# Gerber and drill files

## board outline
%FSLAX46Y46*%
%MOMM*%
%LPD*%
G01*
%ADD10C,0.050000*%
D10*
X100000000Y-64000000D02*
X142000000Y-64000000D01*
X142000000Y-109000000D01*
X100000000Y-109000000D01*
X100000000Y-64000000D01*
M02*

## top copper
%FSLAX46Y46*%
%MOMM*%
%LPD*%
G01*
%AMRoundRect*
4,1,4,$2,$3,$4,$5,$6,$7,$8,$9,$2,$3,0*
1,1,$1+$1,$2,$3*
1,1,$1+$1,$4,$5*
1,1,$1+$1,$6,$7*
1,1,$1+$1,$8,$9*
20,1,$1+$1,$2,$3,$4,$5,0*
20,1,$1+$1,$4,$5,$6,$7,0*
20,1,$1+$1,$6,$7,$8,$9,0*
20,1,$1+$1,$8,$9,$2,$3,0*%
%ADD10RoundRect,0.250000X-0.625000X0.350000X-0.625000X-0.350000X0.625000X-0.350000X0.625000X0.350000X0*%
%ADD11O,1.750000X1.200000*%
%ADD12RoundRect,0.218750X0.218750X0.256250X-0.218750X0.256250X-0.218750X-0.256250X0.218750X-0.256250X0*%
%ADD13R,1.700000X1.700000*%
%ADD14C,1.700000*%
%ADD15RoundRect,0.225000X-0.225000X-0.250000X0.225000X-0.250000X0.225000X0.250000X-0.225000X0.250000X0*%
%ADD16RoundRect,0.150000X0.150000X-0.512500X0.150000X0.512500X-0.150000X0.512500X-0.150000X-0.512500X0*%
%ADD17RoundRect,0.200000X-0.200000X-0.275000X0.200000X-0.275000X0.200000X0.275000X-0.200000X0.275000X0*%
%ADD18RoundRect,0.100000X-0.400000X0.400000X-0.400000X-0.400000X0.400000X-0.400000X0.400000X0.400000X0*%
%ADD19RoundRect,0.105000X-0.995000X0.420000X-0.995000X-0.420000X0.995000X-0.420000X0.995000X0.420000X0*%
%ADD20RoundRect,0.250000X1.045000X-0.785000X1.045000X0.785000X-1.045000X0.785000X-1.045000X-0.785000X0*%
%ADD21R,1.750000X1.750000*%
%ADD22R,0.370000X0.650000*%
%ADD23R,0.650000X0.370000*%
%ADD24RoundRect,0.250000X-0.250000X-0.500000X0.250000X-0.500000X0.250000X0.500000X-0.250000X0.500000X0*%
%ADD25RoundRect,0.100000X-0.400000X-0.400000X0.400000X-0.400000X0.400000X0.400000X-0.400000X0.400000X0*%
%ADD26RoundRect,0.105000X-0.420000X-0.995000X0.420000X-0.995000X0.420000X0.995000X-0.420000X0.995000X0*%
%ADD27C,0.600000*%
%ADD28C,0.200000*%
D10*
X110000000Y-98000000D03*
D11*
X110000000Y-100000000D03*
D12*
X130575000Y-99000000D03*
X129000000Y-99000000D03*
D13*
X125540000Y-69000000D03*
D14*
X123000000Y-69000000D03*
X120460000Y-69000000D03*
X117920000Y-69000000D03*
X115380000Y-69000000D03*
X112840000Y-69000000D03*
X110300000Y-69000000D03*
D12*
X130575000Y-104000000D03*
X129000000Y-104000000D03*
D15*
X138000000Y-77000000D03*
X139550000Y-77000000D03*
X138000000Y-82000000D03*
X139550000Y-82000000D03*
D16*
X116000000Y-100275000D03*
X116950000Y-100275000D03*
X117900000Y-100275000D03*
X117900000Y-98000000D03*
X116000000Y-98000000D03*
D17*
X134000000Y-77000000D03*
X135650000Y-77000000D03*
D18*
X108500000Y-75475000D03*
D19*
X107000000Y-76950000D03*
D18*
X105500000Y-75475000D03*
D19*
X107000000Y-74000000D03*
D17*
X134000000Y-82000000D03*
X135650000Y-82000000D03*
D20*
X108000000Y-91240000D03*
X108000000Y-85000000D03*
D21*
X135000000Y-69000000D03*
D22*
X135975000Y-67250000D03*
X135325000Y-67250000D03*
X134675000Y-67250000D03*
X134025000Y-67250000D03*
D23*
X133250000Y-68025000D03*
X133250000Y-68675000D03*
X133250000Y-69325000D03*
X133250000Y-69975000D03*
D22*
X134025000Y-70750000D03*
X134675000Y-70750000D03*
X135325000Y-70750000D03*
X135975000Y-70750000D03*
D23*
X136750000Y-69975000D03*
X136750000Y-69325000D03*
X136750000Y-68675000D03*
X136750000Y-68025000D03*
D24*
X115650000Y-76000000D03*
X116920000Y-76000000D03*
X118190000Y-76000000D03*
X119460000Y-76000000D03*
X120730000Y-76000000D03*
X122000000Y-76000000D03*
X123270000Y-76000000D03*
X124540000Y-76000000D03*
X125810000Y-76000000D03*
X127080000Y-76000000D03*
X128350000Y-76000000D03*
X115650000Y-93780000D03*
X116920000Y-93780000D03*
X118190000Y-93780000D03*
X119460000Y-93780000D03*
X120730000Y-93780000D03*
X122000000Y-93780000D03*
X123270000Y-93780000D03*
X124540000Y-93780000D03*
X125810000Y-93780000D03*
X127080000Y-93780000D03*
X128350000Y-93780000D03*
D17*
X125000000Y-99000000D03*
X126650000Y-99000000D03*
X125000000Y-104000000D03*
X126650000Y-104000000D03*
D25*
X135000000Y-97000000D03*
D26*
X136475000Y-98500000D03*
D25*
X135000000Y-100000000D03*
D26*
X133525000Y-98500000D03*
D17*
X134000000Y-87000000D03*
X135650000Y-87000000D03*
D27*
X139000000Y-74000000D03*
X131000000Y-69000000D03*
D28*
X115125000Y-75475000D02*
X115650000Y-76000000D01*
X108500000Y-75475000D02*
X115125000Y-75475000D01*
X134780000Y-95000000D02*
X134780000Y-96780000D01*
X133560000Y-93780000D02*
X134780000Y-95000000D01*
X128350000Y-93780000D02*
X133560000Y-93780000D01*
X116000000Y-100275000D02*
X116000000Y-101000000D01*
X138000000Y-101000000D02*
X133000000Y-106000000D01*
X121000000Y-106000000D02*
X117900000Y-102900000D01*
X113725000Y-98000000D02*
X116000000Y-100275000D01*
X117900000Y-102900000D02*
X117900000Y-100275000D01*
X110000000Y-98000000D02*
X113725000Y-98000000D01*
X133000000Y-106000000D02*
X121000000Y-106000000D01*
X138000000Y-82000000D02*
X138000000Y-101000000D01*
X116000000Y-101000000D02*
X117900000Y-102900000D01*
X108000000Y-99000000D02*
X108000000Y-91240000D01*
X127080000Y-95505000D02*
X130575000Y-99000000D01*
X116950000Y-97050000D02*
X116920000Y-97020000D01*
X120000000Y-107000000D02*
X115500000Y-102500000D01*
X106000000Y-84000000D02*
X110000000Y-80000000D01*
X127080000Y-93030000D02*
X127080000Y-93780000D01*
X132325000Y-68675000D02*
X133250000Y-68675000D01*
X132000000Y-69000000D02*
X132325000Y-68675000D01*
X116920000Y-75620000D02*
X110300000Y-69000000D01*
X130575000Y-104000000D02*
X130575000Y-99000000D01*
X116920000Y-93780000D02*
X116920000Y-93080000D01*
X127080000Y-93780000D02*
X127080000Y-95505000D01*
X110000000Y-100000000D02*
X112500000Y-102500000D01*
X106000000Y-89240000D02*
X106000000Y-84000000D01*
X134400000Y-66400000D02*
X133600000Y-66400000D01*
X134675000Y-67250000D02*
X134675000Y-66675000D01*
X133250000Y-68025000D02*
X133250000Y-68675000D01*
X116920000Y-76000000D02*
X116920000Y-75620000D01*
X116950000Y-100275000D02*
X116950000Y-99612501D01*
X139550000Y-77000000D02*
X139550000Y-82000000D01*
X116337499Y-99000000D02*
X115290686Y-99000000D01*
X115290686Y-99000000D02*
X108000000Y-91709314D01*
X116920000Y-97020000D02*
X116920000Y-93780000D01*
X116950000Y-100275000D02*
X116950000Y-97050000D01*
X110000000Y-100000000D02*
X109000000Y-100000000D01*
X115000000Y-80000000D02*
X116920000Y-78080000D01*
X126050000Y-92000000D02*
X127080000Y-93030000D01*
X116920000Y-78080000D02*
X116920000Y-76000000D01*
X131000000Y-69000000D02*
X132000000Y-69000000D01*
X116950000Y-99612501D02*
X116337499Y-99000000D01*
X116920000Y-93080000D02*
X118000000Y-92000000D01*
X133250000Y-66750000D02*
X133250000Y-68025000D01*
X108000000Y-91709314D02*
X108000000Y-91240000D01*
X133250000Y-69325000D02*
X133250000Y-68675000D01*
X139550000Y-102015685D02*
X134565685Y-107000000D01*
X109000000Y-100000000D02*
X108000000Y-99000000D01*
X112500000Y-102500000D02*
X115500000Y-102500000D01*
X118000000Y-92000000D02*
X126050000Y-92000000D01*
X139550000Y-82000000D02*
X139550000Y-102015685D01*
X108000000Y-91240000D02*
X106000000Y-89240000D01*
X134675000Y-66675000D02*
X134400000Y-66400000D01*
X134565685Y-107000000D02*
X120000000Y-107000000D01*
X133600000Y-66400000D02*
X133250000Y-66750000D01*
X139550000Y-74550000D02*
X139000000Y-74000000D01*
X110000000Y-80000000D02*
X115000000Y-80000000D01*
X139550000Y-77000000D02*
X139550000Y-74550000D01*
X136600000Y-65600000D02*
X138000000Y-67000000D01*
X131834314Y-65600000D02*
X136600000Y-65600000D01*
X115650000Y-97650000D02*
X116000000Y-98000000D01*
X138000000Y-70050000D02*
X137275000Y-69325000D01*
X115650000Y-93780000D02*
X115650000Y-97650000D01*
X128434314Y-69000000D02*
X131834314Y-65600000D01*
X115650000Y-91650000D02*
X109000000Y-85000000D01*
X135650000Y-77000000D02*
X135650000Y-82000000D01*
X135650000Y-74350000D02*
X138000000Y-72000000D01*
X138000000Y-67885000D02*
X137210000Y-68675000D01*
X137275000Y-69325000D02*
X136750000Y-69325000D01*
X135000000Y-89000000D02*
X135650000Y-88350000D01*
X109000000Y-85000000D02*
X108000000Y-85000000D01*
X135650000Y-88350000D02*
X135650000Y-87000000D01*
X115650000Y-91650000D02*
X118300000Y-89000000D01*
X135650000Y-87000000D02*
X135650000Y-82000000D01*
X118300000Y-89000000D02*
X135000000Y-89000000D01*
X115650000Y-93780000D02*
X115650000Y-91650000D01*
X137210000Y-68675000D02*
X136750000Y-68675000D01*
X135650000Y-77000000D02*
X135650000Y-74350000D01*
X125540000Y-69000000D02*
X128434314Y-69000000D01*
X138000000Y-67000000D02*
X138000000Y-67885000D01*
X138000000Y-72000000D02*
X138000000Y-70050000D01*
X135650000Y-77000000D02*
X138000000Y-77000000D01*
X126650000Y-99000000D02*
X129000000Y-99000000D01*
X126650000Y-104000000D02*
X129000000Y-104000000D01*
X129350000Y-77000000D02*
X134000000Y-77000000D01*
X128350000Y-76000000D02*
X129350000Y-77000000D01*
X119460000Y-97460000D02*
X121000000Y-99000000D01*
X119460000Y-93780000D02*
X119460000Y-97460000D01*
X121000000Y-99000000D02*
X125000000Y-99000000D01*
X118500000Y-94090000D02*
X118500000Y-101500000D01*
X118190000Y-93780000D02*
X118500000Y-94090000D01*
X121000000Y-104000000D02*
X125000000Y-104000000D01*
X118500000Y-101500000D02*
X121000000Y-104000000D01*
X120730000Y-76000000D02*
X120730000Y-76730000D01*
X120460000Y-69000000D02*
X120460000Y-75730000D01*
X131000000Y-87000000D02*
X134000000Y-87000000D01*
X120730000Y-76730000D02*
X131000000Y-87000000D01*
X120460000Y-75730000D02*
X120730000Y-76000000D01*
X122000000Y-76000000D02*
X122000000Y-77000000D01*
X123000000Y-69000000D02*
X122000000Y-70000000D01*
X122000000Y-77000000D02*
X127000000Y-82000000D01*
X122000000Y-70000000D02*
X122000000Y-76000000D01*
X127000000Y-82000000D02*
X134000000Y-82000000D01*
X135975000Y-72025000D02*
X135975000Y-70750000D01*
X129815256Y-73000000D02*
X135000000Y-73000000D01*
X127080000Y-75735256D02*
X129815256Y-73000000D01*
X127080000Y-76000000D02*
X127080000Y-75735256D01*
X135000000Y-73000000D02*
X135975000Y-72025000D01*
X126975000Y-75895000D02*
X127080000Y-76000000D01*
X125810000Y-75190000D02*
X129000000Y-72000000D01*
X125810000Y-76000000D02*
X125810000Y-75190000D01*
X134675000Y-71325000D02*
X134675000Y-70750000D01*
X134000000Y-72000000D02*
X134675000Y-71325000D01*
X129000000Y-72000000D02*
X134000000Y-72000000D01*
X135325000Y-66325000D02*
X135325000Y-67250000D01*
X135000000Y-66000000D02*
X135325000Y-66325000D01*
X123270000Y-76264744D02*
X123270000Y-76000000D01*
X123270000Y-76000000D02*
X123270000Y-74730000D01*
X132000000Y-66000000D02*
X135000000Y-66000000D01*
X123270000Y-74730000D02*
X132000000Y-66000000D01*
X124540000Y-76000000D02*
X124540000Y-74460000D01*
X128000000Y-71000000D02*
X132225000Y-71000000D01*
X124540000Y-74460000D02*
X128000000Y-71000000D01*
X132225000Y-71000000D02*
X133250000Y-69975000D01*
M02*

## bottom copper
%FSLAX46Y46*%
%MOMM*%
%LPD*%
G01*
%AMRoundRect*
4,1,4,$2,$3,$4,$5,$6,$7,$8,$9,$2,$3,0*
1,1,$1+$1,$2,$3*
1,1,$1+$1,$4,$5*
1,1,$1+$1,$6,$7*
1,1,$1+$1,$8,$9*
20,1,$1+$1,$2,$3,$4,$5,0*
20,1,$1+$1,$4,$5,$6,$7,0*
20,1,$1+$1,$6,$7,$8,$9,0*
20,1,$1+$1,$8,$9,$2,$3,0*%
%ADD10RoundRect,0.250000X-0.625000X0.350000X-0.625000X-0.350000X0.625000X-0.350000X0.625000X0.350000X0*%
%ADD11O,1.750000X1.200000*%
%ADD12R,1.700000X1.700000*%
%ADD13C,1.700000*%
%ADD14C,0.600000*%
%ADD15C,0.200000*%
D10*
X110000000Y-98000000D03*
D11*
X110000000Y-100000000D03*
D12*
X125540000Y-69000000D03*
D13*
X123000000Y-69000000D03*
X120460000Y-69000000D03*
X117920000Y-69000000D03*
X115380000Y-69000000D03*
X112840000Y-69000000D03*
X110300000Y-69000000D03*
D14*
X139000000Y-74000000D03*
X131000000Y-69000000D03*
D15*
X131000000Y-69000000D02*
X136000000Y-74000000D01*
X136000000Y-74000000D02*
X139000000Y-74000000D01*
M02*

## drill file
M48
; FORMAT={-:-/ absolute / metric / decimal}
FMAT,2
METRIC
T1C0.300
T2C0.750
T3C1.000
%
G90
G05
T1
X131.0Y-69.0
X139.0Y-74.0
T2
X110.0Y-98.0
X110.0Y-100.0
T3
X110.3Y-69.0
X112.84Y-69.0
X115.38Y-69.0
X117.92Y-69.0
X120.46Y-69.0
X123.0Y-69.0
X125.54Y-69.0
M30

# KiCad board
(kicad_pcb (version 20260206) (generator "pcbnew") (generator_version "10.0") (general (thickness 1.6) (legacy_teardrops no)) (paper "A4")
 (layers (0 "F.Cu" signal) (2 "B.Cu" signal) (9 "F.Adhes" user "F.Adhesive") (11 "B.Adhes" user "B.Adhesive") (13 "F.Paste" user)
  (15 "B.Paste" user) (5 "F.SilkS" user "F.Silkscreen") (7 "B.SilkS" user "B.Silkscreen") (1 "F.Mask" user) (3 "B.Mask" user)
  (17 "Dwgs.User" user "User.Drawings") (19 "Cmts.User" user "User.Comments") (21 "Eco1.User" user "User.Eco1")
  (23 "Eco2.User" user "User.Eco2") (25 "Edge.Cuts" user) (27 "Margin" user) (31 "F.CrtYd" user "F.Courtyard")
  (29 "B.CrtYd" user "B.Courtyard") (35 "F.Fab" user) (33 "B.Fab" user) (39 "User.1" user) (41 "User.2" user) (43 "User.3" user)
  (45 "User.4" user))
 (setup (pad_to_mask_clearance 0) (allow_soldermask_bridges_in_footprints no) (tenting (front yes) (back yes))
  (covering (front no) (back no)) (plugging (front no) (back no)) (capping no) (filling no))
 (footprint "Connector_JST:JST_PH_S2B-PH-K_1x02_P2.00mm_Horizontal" (layer "F.Cu") (at 110 98 -90)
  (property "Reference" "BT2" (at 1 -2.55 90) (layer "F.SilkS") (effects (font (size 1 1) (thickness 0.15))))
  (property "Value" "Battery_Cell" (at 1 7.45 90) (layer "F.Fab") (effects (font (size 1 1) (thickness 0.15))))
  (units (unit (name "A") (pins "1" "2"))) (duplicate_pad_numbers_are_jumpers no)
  (pad "1" thru_hole roundrect (at 0 0 270) (size 1.2 1.75) (drill 0.75) (layers "*.Cu" "*.Mask") (remove_unused_layers no)
   (roundrect_rratio 0.208333) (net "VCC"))
  (pad "2" thru_hole oval (at 2 0 270) (size 1.2 1.75) (drill 0.75) (layers "*.Cu" "*.Mask") (remove_unused_layers no) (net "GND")))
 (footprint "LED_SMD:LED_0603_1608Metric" (layer "F.Cu") (at 129.7875 99 180)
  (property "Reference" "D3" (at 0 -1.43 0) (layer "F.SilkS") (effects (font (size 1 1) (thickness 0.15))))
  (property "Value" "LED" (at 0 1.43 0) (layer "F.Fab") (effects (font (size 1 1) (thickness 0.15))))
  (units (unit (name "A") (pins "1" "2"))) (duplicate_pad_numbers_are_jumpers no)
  (pad "1" smd roundrect (at -0.7875 0 180) (size 0.875 0.95) (layers "F.Cu" "F.Mask" "F.Paste") (roundrect_rratio 0.25) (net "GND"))
  (pad "2" smd roundrect (at 0.7875 0 180) (size 0.875 0.95) (layers "F.Cu" "F.Mask" "F.Paste") (roundrect_rratio 0.25) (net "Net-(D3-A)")))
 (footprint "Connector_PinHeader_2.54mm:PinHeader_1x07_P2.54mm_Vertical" (layer "F.Cu") (at 125.54 69 -90)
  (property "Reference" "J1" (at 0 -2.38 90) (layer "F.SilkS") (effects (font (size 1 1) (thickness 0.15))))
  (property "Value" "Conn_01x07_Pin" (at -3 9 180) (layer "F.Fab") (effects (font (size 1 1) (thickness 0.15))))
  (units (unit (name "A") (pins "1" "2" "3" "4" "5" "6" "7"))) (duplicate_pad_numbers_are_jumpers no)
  (pad "1" thru_hole rect (at 0 0 270) (size 1.7 1.7) (drill 1) (layers "*.Cu" "*.Mask") (remove_unused_layers no) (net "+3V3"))
  (pad "2" thru_hole circle (at 0 2.54 270) (size 1.7 1.7) (drill 1) (layers "*.Cu" "*.Mask") (remove_unused_layers no)
   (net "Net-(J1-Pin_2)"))
  (pad "3" thru_hole circle (at 0 5.08 270) (size 1.7 1.7) (drill 1) (layers "*.Cu" "*.Mask") (remove_unused_layers no)
   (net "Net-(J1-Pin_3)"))
  (pad "4" thru_hole circle (at 0 7.62 270) (size 1.7 1.7) (drill 1) (layers "*.Cu" "*.Mask") (remove_unused_layers no)
   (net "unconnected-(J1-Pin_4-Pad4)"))
  (pad "5" thru_hole circle (at 0 10.16 270) (size 1.7 1.7) (drill 1) (layers "*.Cu" "*.Mask") (remove_unused_layers no)
   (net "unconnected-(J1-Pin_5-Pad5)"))
  (pad "6" thru_hole circle (at 0 12.7 270) (size 1.7 1.7) (drill 1) (layers "*.Cu" "*.Mask") (remove_unused_layers no)
   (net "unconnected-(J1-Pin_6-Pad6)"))
  (pad "7" thru_hole circle (at 0 15.24 270) (size 1.7 1.7) (drill 1) (layers "*.Cu" "*.Mask") (remove_unused_layers no) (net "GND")))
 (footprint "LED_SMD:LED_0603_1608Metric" (layer "F.Cu") (at 129.7875 104 180)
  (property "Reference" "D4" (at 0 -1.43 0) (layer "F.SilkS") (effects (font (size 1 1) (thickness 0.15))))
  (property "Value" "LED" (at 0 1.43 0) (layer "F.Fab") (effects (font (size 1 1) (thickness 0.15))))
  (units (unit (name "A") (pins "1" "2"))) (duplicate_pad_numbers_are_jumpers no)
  (pad "1" smd roundrect (at -0.7875 0 180) (size 0.875 0.95) (layers "F.Cu" "F.Mask" "F.Paste") (roundrect_rratio 0.25) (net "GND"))
  (pad "2" smd roundrect (at 0.7875 0 180) (size 0.875 0.95) (layers "F.Cu" "F.Mask" "F.Paste") (roundrect_rratio 0.25) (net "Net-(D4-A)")))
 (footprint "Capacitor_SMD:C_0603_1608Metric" (layer "F.Cu") (at 138.775 77)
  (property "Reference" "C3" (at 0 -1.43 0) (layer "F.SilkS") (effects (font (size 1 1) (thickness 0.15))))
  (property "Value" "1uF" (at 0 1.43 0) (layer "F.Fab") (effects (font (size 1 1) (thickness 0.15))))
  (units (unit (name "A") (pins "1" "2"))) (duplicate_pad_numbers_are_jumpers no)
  (pad "1" smd roundrect (at -0.775 0) (size 0.9 0.95) (layers "F.Cu" "F.Mask" "F.Paste") (roundrect_rratio 0.25) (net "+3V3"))
  (pad "2" smd roundrect (at 0.775 0) (size 0.9 0.95) (layers "F.Cu" "F.Mask" "F.Paste") (roundrect_rratio 0.25) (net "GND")))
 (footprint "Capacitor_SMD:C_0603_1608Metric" (layer "F.Cu") (at 138.775 82)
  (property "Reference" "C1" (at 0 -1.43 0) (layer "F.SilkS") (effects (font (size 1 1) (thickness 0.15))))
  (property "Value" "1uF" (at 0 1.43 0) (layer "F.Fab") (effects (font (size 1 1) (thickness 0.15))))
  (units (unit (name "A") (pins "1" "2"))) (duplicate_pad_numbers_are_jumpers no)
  (pad "1" smd roundrect (at -0.775 0) (size 0.9 0.95) (layers "F.Cu" "F.Mask" "F.Paste") (roundrect_rratio 0.25) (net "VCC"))
  (pad "2" smd roundrect (at 0.775 0) (size 0.9 0.95) (layers "F.Cu" "F.Mask" "F.Paste") (roundrect_rratio 0.25) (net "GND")))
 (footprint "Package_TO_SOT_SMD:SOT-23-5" (layer "F.Cu") (at 116.95 99.1375 90)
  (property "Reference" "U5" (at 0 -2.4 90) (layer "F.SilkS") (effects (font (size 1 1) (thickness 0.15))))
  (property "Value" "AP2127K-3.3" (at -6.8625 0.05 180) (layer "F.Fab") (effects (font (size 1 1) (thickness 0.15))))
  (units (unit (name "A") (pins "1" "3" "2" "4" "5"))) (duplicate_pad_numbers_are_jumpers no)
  (pad "1" smd roundrect (at -1.1375 -0.95 90) (size 1.325 0.6) (layers "F.Cu" "F.Mask" "F.Paste") (roundrect_rratio 0.25) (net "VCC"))
  (pad "2" smd roundrect (at -1.1375 0 90) (size 1.325 0.6) (layers "F.Cu" "F.Mask" "F.Paste") (roundrect_rratio 0.25) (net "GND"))
  (pad "3" smd roundrect (at -1.1375 0.95 90) (size 1.325 0.6) (layers "F.Cu" "F.Mask" "F.Paste") (roundrect_rratio 0.25) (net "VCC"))
  (pad "4" smd roundrect (at 1.1375 0.95 90) (size 1.325 0.6) (layers "F.Cu" "F.Mask" "F.Paste") (roundrect_rratio 0.25)
   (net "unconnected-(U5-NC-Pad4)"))
  (pad "5" smd roundrect (at 1.1375 -0.95 90) (size 1.325 0.6) (layers "F.Cu" "F.Mask" "F.Paste") (roundrect_rratio 0.25) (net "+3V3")))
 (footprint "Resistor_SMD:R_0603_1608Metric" (layer "F.Cu") (at 134.825 77)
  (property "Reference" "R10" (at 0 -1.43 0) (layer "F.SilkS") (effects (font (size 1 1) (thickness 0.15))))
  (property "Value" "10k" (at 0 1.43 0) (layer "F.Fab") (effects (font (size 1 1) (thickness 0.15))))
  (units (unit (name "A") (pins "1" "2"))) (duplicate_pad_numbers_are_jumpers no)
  (pad "1" smd roundrect (at -0.825 0) (size 0.8 0.95) (layers "F.Cu" "F.Mask" "F.Paste") (roundrect_rratio 0.25) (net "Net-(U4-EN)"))
  (pad "2" smd roundrect (at 0.825 0) (size 0.8 0.95) (layers "F.Cu" "F.Mask" "F.Paste") (roundrect_rratio 0.25) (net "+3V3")))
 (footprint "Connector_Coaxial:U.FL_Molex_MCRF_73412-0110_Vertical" (layer "F.Cu") (at 107 75.475 90)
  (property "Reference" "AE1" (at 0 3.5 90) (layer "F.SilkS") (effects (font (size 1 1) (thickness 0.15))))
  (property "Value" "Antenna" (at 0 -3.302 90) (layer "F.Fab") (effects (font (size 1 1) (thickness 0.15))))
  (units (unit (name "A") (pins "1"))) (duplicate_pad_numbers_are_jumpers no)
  (pad "1" smd roundrect (at 0 1.5 270) (size 1 1) (layers "F.Cu" "F.Mask" "F.Paste") (roundrect_rratio 0.1) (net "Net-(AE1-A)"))
  (pad "2" smd roundrect (at -1.475 0 270) (size 1.05 2.2) (layers "F.Cu" "F.Mask" "F.Paste") (roundrect_rratio 0.1))
  (pad "2" smd roundrect (at 0 -1.5 270) (size 1 1) (layers "F.Cu" "F.Mask" "F.Paste") (roundrect_rratio 0.1))
  (pad "2" smd roundrect (at 1.475 0 270) (size 1.05 2.2) (layers "F.Cu" "F.Mask" "F.Paste") (roundrect_rratio 0.1)))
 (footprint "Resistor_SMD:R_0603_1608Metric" (layer "F.Cu") (at 134.825 82)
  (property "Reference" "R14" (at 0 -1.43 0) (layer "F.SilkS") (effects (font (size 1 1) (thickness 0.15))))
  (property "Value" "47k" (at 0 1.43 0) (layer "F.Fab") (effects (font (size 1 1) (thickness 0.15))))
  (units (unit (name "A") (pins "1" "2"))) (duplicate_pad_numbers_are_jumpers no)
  (pad "1" smd roundrect (at -0.825 0) (size 0.8 0.95) (layers "F.Cu" "F.Mask" "F.Paste") (roundrect_rratio 0.25) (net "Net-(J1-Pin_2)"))
  (pad "2" smd roundrect (at 0.825 0) (size 0.8 0.95) (layers "F.Cu" "F.Mask" "F.Paste") (roundrect_rratio 0.25) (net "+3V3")))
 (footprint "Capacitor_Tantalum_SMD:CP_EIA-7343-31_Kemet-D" (layer "F.Cu") (at 108 88.12 90)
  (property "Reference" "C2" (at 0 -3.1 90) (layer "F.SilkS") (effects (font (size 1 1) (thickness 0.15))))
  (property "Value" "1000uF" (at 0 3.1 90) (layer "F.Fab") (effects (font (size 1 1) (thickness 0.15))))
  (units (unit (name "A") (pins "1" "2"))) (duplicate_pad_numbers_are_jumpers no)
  (pad "1" smd roundrect (at -3.12 0 90) (size 2.07 2.59) (layers "F.Cu" "F.Mask" "F.Paste") (roundrect_rratio 0.120773) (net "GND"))
  (pad "2" smd roundrect (at 3.12 0 90) (size 2.07 2.59) (layers "F.Cu" "F.Mask" "F.Paste") (roundrect_rratio 0.120773) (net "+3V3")))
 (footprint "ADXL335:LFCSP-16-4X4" (layer "F.Cu") (at 135 69 -90)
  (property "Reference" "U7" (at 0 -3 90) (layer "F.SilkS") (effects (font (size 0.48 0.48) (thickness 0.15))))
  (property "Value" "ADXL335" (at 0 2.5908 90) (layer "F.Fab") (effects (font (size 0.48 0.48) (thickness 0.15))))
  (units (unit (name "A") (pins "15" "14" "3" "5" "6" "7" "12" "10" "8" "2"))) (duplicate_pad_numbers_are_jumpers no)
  (pad "0" smd rect (at 0 0 270) (size 1.75 1.75) (layers "F.Cu" "F.Mask") (solder_mask_margin 0.102))
  (pad "1" smd rect (at -1.75 -0.975 270) (size 0.65 0.37) (layers "F.Cu" "F.Mask" "F.Paste") (solder_mask_margin 0.102))
  (pad "2" smd rect (at -1.75 -0.325 270) (size 0.65 0.37) (layers "F.Cu" "F.Mask" "F.Paste") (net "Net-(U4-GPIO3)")
   (solder_mask_margin 0.102))
  (pad "3" smd rect (at -1.75 0.325 270) (size 0.65 0.37) (layers "F.Cu" "F.Mask" "F.Paste") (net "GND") (solder_mask_margin 0.102))
  (pad "4" smd rect (at -1.75 0.975 270) (size 0.65 0.37) (layers "F.Cu" "F.Mask" "F.Paste") (solder_mask_margin 0.102))
  (pad "5" smd rect (at -0.975 1.75 270) (size 0.37 0.65) (layers "F.Cu" "F.Mask" "F.Paste") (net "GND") (solder_mask_margin 0.102))
  (pad "6" smd rect (at -0.325 1.75 270) (size 0.37 0.65) (layers "F.Cu" "F.Mask" "F.Paste") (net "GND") (solder_mask_margin 0.102))
  (pad "7" smd rect (at 0.325 1.75 270) (size 0.37 0.65) (layers "F.Cu" "F.Mask" "F.Paste") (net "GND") (solder_mask_margin 0.102))
  (pad "8" smd rect (at 0.975 1.75 270) (size 0.37 0.65) (layers "F.Cu" "F.Mask" "F.Paste") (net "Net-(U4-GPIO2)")
   (solder_mask_margin 0.102))
  (pad "9" smd rect (at 1.75 0.975 270) (size 0.65 0.37) (layers "F.Cu" "F.Mask" "F.Paste") (solder_mask_margin 0.102))
  (pad "10" smd rect (at 1.75 0.325 270) (size 0.65 0.37) (layers "F.Cu" "F.Mask" "F.Paste") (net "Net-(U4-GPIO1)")
   (solder_mask_margin 0.102))
  (pad "11" smd rect (at 1.75 -0.325 270) (size 0.65 0.37) (layers "F.Cu" "F.Mask" "F.Paste") (solder_mask_margin 0.102))
  (pad "12" smd rect (at 1.75 -0.975 270) (size 0.65 0.37) (layers "F.Cu" "F.Mask" "F.Paste") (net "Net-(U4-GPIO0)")
   (solder_mask_margin 0.102))
  (pad "13" smd rect (at 0.975 -1.75 270) (size 0.37 0.65) (layers "F.Cu" "F.Mask" "F.Paste") (solder_mask_margin 0.102))
  (pad "14" smd rect (at 0.325 -1.75 270) (size 0.37 0.65) (layers "F.Cu" "F.Mask" "F.Paste") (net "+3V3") (solder_mask_margin 0.102))
  (pad "15" smd rect (at -0.325 -1.75 270) (size 0.37 0.65) (layers "F.Cu" "F.Mask" "F.Paste") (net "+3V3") (solder_mask_margin 0.102))
  (pad "16" smd rect (at -0.975 -1.75 270) (size 0.37 0.65) (layers "F.Cu" "F.Mask" "F.Paste") (solder_mask_margin 0.102)))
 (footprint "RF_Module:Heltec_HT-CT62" (layer "F.Cu") (at 122 84.89)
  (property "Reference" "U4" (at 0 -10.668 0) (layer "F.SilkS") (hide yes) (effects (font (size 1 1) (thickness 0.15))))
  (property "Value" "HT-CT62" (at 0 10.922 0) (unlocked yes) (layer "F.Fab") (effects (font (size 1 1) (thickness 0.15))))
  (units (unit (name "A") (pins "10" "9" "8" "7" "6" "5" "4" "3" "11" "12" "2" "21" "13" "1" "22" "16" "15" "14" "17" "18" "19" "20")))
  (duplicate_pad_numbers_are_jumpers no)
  (pad "1" smd roundrect (at -6.35 -8.89) (size 1 1.5) (layers "F.Cu" "F.Mask" "F.Paste") (roundrect_rratio 0.25) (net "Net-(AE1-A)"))
  (pad "2" smd roundrect (at -5.08 -8.89) (size 1 1.5) (layers "F.Cu" "F.Mask" "F.Paste") (roundrect_rratio 0.25) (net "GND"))
  (pad "3" smd roundrect (at -3.81 -8.89) (size 1 1.5) (layers "F.Cu" "F.Mask" "F.Paste") (roundrect_rratio 0.25)
   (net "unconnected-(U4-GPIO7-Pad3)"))
  (pad "4" smd roundrect (at -2.54 -8.89) (size 1 1.5) (layers "F.Cu" "F.Mask" "F.Paste") (roundrect_rratio 0.25)
   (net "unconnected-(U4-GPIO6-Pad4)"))
  (pad "5" smd roundrect (at -1.27 -8.89) (size 1 1.5) (layers "F.Cu" "F.Mask" "F.Paste") (roundrect_rratio 0.25) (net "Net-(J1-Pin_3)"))
  (pad "6" smd roundrect (at 0 -8.89) (size 1 1.5) (layers "F.Cu" "F.Mask" "F.Paste") (roundrect_rratio 0.25) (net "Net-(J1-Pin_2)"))
  (pad "7" smd roundrect (at 1.27 -8.89) (size 1 1.5) (layers "F.Cu" "F.Mask" "F.Paste") (roundrect_rratio 0.25) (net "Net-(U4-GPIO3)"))
  (pad "8" smd roundrect (at 2.54 -8.89) (size 1 1.5) (layers "F.Cu" "F.Mask" "F.Paste") (roundrect_rratio 0.25) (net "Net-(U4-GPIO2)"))
  (pad "9" smd roundrect (at 3.81 -8.89) (size 1 1.5) (layers "F.Cu" "F.Mask" "F.Paste") (roundrect_rratio 0.25) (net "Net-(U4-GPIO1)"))
  (pad "10" smd roundrect (at 5.08 -8.89) (size 1 1.5) (layers "F.Cu" "F.Mask" "F.Paste") (roundrect_rratio 0.25) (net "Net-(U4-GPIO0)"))
  (pad "11" smd roundrect (at 6.35 -8.89) (size 1 1.5) (layers "F.Cu" "F.Mask" "F.Paste") (roundrect_rratio 0.25) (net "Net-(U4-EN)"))
  (pad "12" smd roundrect (at -6.35 8.89) (size 1 1.5) (layers "F.Cu" "F.Mask" "F.Paste") (roundrect_rratio 0.25) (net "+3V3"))
  (pad "13" smd roundrect (at -5.08 8.89) (size 1 1.5) (layers "F.Cu" "F.Mask" "F.Paste") (roundrect_rratio 0.25) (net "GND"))
  (pad "14" smd roundrect (at -3.81 8.89) (size 1 1.5) (layers "F.Cu" "F.Mask" "F.Paste") (roundrect_rratio 0.25) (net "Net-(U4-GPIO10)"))
  (pad "15" smd roundrect (at -2.54 8.89) (size 1 1.5) (layers "F.Cu" "F.Mask" "F.Paste") (roundrect_rratio 0.25) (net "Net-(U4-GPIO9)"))
  (pad "16" smd roundrect (at -1.27 8.89) (size 1 1.5) (layers "F.Cu" "F.Mask" "F.Paste") (roundrect_rratio 0.25)
   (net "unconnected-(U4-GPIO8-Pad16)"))
  (pad "17" smd roundrect (at 0 8.89) (size 1 1.5) (layers "F.Cu" "F.Mask" "F.Paste") (roundrect_rratio 0.25)
   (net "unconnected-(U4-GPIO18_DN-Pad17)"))
  (pad "18" smd roundrect (at 1.27 8.89) (size 1 1.5) (layers "F.Cu" "F.Mask" "F.Paste") (roundrect_rratio 0.25)
   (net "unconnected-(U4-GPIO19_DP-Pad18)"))
  (pad "19" smd roundrect (at 2.54 8.89) (size 1 1.5) (layers "F.Cu" "F.Mask" "F.Paste") (roundrect_rratio 0.25)
   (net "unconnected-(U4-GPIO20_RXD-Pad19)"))
  (pad "20" smd roundrect (at 3.81 8.89) (size 1 1.5) (layers "F.Cu" "F.Mask" "F.Paste") (roundrect_rratio 0.25)
   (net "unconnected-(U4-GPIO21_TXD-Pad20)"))
  (pad "21" smd roundrect (at 5.08 8.89) (size 1 1.5) (layers "F.Cu" "F.Mask" "F.Paste") (roundrect_rratio 0.25) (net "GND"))
  (pad "22" smd roundrect (at 6.35 8.89) (size 1 1.5) (layers "F.Cu" "F.Mask" "F.Paste") (roundrect_rratio 0.25) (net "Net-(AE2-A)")))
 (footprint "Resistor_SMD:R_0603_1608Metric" (layer "F.Cu") (at 125.825 99)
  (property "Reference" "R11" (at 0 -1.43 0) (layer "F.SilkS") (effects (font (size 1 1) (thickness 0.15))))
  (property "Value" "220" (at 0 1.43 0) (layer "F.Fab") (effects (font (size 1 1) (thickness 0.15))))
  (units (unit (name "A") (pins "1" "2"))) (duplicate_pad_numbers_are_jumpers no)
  (pad "1" smd roundrect (at -0.825 0) (size 0.8 0.95) (layers "F.Cu" "F.Mask" "F.Paste") (roundrect_rratio 0.25) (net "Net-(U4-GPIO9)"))
  (pad "2" smd roundrect (at 0.825 0) (size 0.8 0.95) (layers "F.Cu" "F.Mask" "F.Paste") (roundrect_rratio 0.25) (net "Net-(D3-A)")))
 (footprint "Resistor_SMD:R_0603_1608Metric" (layer "F.Cu") (at 125.825 104)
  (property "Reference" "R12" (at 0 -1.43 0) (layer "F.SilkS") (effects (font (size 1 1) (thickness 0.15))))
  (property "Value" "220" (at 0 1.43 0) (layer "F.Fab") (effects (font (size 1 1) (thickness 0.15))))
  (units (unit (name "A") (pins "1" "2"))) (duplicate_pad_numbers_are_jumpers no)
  (pad "1" smd roundrect (at -0.825 0) (size 0.8 0.95) (layers "F.Cu" "F.Mask" "F.Paste") (roundrect_rratio 0.25) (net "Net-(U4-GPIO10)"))
  (pad "2" smd roundrect (at 0.825 0) (size 0.8 0.95) (layers "F.Cu" "F.Mask" "F.Paste") (roundrect_rratio 0.25) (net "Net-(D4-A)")))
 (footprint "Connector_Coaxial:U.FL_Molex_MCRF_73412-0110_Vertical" (layer "F.Cu") (at 135 98.5 180)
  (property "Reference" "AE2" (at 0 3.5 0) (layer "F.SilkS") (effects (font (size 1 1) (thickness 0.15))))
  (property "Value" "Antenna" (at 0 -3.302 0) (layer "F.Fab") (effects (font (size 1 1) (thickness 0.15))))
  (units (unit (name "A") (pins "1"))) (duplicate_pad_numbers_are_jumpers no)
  (pad "1" smd roundrect (at 0 1.5) (size 1 1) (layers "F.Cu" "F.Mask" "F.Paste") (roundrect_rratio 0.1) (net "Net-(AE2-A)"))
  (pad "2" smd roundrect (at -1.475 0) (size 1.05 2.2) (layers "F.Cu" "F.Mask" "F.Paste") (roundrect_rratio 0.1))
  (pad "2" smd roundrect (at 0 -1.5) (size 1 1) (layers "F.Cu" "F.Mask" "F.Paste") (roundrect_rratio 0.1))
  (pad "2" smd roundrect (at 1.475 0) (size 1.05 2.2) (layers "F.Cu" "F.Mask" "F.Paste") (roundrect_rratio 0.1)))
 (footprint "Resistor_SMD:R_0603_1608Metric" (layer "F.Cu") (at 134.825 87)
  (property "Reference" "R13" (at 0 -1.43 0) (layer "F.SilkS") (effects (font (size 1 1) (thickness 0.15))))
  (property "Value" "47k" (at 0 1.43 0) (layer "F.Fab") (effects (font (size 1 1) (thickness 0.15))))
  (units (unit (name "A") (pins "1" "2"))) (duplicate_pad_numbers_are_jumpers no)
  (pad "1" smd roundrect (at -0.825 0) (size 0.8 0.95) (layers "F.Cu" "F.Mask" "F.Paste") (roundrect_rratio 0.25) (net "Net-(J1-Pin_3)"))
  (pad "2" smd roundrect (at 0.825 0) (size 0.8 0.95) (layers "F.Cu" "F.Mask" "F.Paste") (roundrect_rratio 0.25) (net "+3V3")))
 (gr_rect (start 100 64) (end 142 109) (stroke (width 0.05) (type default)) (fill no) (layer "Edge.Cuts"))
 (segment (start 115.125 75.475) (end 115.65 76) (width 0.2) (layer "F.Cu") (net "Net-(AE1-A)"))
 (segment (start 108.5 75.475) (end 115.125 75.475) (width 0.2) (layer "F.Cu") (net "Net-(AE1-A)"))
 (segment (start 134.78 95) (end 134.78 96.78) (width 0.2) (layer "F.Cu") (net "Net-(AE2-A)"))
 (segment (start 133.56 93.78) (end 134.78 95) (width 0.2) (layer "F.Cu") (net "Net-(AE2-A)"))
 (segment (start 128.35 93.78) (end 133.56 93.78) (width 0.2) (layer "F.Cu") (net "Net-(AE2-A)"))
 (segment (start 116 100.275) (end 116 101) (width 0.2) (layer "F.Cu") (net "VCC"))
 (segment (start 138 101) (end 133 106) (width 0.2) (layer "F.Cu") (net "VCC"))
 (segment (start 121 106) (end 117.9 102.9) (width 0.2) (layer "F.Cu") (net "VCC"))
 (segment (start 113.725 98) (end 116 100.275) (width 0.2) (layer "F.Cu") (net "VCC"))
 (segment (start 117.9 102.9) (end 117.9 100.275) (width 0.2) (layer "F.Cu") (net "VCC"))
 (segment (start 110 98) (end 113.725 98) (width 0.2) (layer "F.Cu") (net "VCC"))
 (segment (start 133 106) (end 121 106) (width 0.2) (layer "F.Cu") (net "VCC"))
 (segment (start 138 82) (end 138 101) (width 0.2) (layer "F.Cu") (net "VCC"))
 (segment (start 116 101) (end 117.9 102.9) (width 0.2) (layer "F.Cu") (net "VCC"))
 (segment (start 108 99) (end 108 91.24) (width 0.2) (layer "F.Cu") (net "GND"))
 (segment (start 127.08 95.505) (end 130.575 99) (width 0.2) (layer "F.Cu") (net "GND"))
 (segment (start 116.95 97.05) (end 116.92 97.02) (width 0.2) (layer "F.Cu") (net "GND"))
 (segment (start 120 107) (end 115.5 102.5) (width 0.2) (layer "F.Cu") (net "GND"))
 (segment (start 106 84) (end 110 80) (width 0.2) (layer "F.Cu") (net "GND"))
 (segment (start 127.08 93.03) (end 127.08 93.78) (width 0.2) (layer "F.Cu") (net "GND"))
 (segment (start 132.325 68.675) (end 133.25 68.675) (width 0.2) (layer "F.Cu") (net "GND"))
 (segment (start 132 69) (end 132.325 68.675) (width 0.2) (layer "F.Cu") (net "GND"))
 (segment (start 116.92 75.62) (end 110.3 69) (width 0.2) (layer "F.Cu") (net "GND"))
 (segment (start 130.575 104) (end 130.575 99) (width 0.2) (layer "F.Cu") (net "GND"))
 (segment (start 116.92 93.78) (end 116.92 93.08) (width 0.2) (layer "F.Cu") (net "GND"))
 (segment (start 127.08 93.78) (end 127.08 95.505) (width 0.2) (layer "F.Cu") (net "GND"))
 (segment (start 110 100) (end 112.5 102.5) (width 0.2) (layer "F.Cu") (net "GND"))
 (segment (start 106 89.24) (end 106 84) (width 0.2) (layer "F.Cu") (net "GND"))
 (segment (start 134.4 66.4) (end 133.6 66.4) (width 0.2) (layer "F.Cu") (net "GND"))
 (segment (start 134.675 67.25) (end 134.675 66.675) (width 0.2) (layer "F.Cu") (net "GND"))
 (segment (start 133.25 68.025) (end 133.25 68.675) (width 0.2) (layer "F.Cu") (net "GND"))
 (segment (start 116.92 76) (end 116.92 75.62) (width 0.2) (layer "F.Cu") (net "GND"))
 (segment (start 116.95 100.275) (end 116.95 99.612501) (width 0.2) (layer "F.Cu") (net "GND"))
 (segment (start 139.55 77) (end 139.55 82) (width 0.2) (layer "F.Cu") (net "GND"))
 (segment (start 116.337499 99) (end 115.290686 99) (width 0.2) (layer "F.Cu") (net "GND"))
 (segment (start 115.290686 99) (end 108 91.709314) (width 0.2) (layer "F.Cu") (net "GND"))
 (segment (start 116.92 97.02) (end 116.92 93.78) (width 0.2) (layer "F.Cu") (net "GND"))
 (segment (start 116.95 100.275) (end 116.95 97.05) (width 0.2) (layer "F.Cu") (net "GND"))
 (segment (start 110 100) (end 109 100) (width 0.2) (layer "F.Cu") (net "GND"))
 (segment (start 115 80) (end 116.92 78.08) (width 0.2) (layer "F.Cu") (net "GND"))
 (segment (start 126.05 92) (end 127.08 93.03) (width 0.2) (layer "F.Cu") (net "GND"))
 (segment (start 116.92 78.08) (end 116.92 76) (width 0.2) (layer "F.Cu") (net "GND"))
 (segment (start 131 69) (end 132 69) (width 0.2) (layer "F.Cu") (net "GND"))
 (segment (start 116.95 99.612501) (end 116.337499 99) (width 0.2) (layer "F.Cu") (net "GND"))
 (segment (start 116.92 93.08) (end 118 92) (width 0.2) (layer "F.Cu") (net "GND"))
 (segment (start 133.25 66.75) (end 133.25 68.025) (width 0.2) (layer "F.Cu") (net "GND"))
 (segment (start 108 91.709314) (end 108 91.24) (width 0.2) (layer "F.Cu") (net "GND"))
 (segment (start 133.25 69.325) (end 133.25 68.675) (width 0.2) (layer "F.Cu") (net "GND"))
 (segment (start 139.55 102.015685) (end 134.565685 107) (width 0.2) (layer "F.Cu") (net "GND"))
 (segment (start 109 100) (end 108 99) (width 0.2) (layer "F.Cu") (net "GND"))
 (segment (start 112.5 102.5) (end 115.5 102.5) (width 0.2) (layer "F.Cu") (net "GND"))
 (segment (start 118 92) (end 126.05 92) (width 0.2) (layer "F.Cu") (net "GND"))
 (segment (start 139.55 82) (end 139.55 102.015685) (width 0.2) (layer "F.Cu") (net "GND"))
 (segment (start 108 91.24) (end 106 89.24) (width 0.2) (layer "F.Cu") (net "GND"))
 (segment (start 134.675 66.675) (end 134.4 66.4) (width 0.2) (layer "F.Cu") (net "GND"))
 (segment (start 134.565685 107) (end 120 107) (width 0.2) (layer "F.Cu") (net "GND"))
 (segment (start 133.6 66.4) (end 133.25 66.75) (width 0.2) (layer "F.Cu") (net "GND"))
 (segment (start 139.55 74.55) (end 139 74) (width 0.2) (layer "F.Cu") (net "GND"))
 (segment (start 110 80) (end 115 80) (width 0.2) (layer "F.Cu") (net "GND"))
 (segment (start 139.55 77) (end 139.55 74.55) (width 0.2) (layer "F.Cu") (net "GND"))
 (via (at 139 74) (size 0.6) (drill 0.3) (layers "F.Cu" "B.Cu") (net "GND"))
 (via (at 131 69) (size 0.6) (drill 0.3) (layers "F.Cu" "B.Cu") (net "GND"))
 (segment (start 131 69) (end 136 74) (width 0.2) (layer "B.Cu") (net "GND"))
 (segment (start 136 74) (end 139 74) (width 0.2) (layer "B.Cu") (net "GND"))
 (segment (start 136.6 65.6) (end 138 67) (width 0.2) (layer "F.Cu") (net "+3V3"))
 (segment (start 131.834314 65.6) (end 136.6 65.6) (width 0.2) (layer "F.Cu") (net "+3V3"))
 (segment (start 115.65 97.65) (end 116 98) (width 0.2) (layer "F.Cu") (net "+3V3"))
 (segment (start 138 70.05) (end 137.275 69.325) (width 0.2) (layer "F.Cu") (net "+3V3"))
 (segment (start 115.65 93.78) (end 115.65 97.65) (width 0.2) (layer "F.Cu") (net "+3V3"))
 (segment (start 128.434314 69) (end 131.834314 65.6) (width 0.2) (layer "F.Cu") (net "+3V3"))
 (segment (start 115.65 91.65) (end 109 85) (width 0.2) (layer "F.Cu") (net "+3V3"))
 (segment (start 135.65 77) (end 135.65 82) (width 0.2) (layer "F.Cu") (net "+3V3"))
 (segment (start 135.65 74.35) (end 138 72) (width 0.2) (layer "F.Cu") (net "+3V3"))
 (segment (start 138 67.885) (end 137.21 68.675) (width 0.2) (layer "F.Cu") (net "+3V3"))
 (segment (start 137.275 69.325) (end 136.75 69.325) (width 0.2) (layer "F.Cu") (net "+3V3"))
 (segment (start 135 89) (end 135.65 88.35) (width 0.2) (layer "F.Cu") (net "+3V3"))
 (segment (start 109 85) (end 108 85) (width 0.2) (layer "F.Cu") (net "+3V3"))
 (segment (start 135.65 88.35) (end 135.65 87) (width 0.2) (layer "F.Cu") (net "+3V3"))
 (segment (start 115.65 91.65) (end 118.3 89) (width 0.2) (layer "F.Cu") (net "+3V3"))
 (segment (start 135.65 87) (end 135.65 82) (width 0.2) (layer "F.Cu") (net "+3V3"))
 (segment (start 118.3 89) (end 135 89) (width 0.2) (layer "F.Cu") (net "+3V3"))
 (segment (start 115.65 93.78) (end 115.65 91.65) (width 0.2) (layer "F.Cu") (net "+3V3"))
 (segment (start 137.21 68.675) (end 136.75 68.675) (width 0.2) (layer "F.Cu") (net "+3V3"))
 (segment (start 135.65 77) (end 135.65 74.35) (width 0.2) (layer "F.Cu") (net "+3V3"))
 (segment (start 125.54 69) (end 128.434314 69) (width 0.2) (layer "F.Cu") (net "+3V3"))
 (segment (start 138 67) (end 138 67.885) (width 0.2) (layer "F.Cu") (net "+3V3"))
 (segment (start 138 72) (end 138 70.05) (width 0.2) (layer "F.Cu") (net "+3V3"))
 (segment (start 135.65 77) (end 138 77) (width 0.2) (layer "F.Cu") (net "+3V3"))
 (segment (start 126.65 99) (end 129 99) (width 0.2) (layer "F.Cu") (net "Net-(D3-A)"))
 (segment (start 126.65 104) (end 129 104) (width 0.2) (layer "F.Cu") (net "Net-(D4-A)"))
 (segment (start 129.35 77) (end 134 77) (width 0.2) (layer "F.Cu") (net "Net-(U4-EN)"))
 (segment (start 128.35 76) (end 129.35 77) (width 0.2) (layer "F.Cu") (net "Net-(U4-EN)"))
 (segment (start 119.46 97.46) (end 121 99) (width 0.2) (layer "F.Cu") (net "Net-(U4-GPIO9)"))
 (segment (start 119.46 93.78) (end 119.46 97.46) (width 0.2) (layer "F.Cu") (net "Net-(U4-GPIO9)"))
 (segment (start 121 99) (end 125 99) (width 0.2) (layer "F.Cu") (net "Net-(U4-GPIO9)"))
 (segment (start 118.5 94.09) (end 118.5 101.5) (width 0.2) (layer "F.Cu") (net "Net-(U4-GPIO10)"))
 (segment (start 118.19 93.78) (end 118.5 94.09) (width 0.2) (layer "F.Cu") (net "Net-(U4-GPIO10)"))
 (segment (start 121 104) (end 125 104) (width 0.2) (layer "F.Cu") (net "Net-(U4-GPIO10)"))
 (segment (start 118.5 101.5) (end 121 104) (width 0.2) (layer "F.Cu") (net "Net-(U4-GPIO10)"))
 (segment (start 120.73 76) (end 120.73 76.73) (width 0.2) (layer "F.Cu") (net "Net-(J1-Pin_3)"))
 (segment (start 120.46 69) (end 120.46 75.73) (width 0.2) (layer "F.Cu") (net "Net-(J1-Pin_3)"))
 (segment (start 131 87) (end 134 87) (width 0.2) (layer "F.Cu") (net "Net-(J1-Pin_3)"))
 (segment (start 120.73 76.73) (end 131 87) (width 0.2) (layer "F.Cu") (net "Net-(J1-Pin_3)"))
 (segment (start 120.46 75.73) (end 120.73 76) (width 0.2) (layer "F.Cu") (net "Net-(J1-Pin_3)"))
 (segment (start 122 76) (end 122 77) (width 0.2) (layer "F.Cu") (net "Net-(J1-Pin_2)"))
 (segment (start 123 69) (end 122 70) (width 0.2) (layer "F.Cu") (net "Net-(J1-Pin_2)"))
 (segment (start 122 77) (end 127 82) (width 0.2) (layer "F.Cu") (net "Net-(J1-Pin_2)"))
 (segment (start 122 70) (end 122 76) (width 0.2) (layer "F.Cu") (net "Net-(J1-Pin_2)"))
 (segment (start 127 82) (end 134 82) (width 0.2) (layer "F.Cu") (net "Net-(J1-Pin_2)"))
 (segment (start 135.975 72.025) (end 135.975 70.75) (width 0.2) (layer "F.Cu") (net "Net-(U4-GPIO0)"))
 (segment (start 129.815256 73) (end 135 73) (width 0.2) (layer "F.Cu") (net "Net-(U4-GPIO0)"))
 (segment (start 127.08 75.735256) (end 129.815256 73) (width 0.2) (layer "F.Cu") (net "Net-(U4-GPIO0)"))
 (segment (start 127.08 76) (end 127.08 75.735256) (width 0.2) (layer "F.Cu") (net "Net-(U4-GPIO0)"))
 (segment (start 135 73) (end 135.975 72.025) (width 0.2) (layer "F.Cu") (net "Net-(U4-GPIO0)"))
 (segment (start 126.975 75.895) (end 127.08 76) (width 0.2) (layer "F.Cu") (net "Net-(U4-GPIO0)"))
 (segment (start 125.81 75.19) (end 129 72) (width 0.2) (layer "F.Cu") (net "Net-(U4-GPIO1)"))
 (segment (start 125.81 76) (end 125.81 75.19) (width 0.2) (layer "F.Cu") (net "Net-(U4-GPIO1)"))
 (segment (start 134.675 71.325) (end 134.675 70.75) (width 0.2) (layer "F.Cu") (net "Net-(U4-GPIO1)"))
 (segment (start 134 72) (end 134.675 71.325) (width 0.2) (layer "F.Cu") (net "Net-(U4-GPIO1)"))
 (segment (start 129 72) (end 134 72) (width 0.2) (layer "F.Cu") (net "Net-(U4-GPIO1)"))
 (segment (start 135.325 66.325) (end 135.325 67.25) (width 0.2) (layer "F.Cu") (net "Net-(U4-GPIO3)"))
 (segment (start 135 66) (end 135.325 66.325) (width 0.2) (layer "F.Cu") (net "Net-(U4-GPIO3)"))
 (segment (start 123.27 76.264744) (end 123.27 76) (width 0.2) (layer "F.Cu") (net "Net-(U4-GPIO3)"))
 (segment (start 123.27 76) (end 123.27 74.73) (width 0.2) (layer "F.Cu") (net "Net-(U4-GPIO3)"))
 (segment (start 132 66) (end 135 66) (width 0.2) (layer "F.Cu") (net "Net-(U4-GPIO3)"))
 (segment (start 123.27 74.73) (end 132 66) (width 0.2) (layer "F.Cu") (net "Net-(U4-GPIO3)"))
 (segment (start 124.54 76) (end 124.54 74.46) (width 0.2) (layer "F.Cu") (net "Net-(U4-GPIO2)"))
 (segment (start 128 71) (end 132.225 71) (width 0.2) (layer "F.Cu") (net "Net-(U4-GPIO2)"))
 (segment (start 124.54 74.46) (end 128 71) (width 0.2) (layer "F.Cu") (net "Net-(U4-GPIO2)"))
 (segment (start 132.225 71) (end 133.25 69.975) (width 0.2) (layer "F.Cu") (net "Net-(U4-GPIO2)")))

